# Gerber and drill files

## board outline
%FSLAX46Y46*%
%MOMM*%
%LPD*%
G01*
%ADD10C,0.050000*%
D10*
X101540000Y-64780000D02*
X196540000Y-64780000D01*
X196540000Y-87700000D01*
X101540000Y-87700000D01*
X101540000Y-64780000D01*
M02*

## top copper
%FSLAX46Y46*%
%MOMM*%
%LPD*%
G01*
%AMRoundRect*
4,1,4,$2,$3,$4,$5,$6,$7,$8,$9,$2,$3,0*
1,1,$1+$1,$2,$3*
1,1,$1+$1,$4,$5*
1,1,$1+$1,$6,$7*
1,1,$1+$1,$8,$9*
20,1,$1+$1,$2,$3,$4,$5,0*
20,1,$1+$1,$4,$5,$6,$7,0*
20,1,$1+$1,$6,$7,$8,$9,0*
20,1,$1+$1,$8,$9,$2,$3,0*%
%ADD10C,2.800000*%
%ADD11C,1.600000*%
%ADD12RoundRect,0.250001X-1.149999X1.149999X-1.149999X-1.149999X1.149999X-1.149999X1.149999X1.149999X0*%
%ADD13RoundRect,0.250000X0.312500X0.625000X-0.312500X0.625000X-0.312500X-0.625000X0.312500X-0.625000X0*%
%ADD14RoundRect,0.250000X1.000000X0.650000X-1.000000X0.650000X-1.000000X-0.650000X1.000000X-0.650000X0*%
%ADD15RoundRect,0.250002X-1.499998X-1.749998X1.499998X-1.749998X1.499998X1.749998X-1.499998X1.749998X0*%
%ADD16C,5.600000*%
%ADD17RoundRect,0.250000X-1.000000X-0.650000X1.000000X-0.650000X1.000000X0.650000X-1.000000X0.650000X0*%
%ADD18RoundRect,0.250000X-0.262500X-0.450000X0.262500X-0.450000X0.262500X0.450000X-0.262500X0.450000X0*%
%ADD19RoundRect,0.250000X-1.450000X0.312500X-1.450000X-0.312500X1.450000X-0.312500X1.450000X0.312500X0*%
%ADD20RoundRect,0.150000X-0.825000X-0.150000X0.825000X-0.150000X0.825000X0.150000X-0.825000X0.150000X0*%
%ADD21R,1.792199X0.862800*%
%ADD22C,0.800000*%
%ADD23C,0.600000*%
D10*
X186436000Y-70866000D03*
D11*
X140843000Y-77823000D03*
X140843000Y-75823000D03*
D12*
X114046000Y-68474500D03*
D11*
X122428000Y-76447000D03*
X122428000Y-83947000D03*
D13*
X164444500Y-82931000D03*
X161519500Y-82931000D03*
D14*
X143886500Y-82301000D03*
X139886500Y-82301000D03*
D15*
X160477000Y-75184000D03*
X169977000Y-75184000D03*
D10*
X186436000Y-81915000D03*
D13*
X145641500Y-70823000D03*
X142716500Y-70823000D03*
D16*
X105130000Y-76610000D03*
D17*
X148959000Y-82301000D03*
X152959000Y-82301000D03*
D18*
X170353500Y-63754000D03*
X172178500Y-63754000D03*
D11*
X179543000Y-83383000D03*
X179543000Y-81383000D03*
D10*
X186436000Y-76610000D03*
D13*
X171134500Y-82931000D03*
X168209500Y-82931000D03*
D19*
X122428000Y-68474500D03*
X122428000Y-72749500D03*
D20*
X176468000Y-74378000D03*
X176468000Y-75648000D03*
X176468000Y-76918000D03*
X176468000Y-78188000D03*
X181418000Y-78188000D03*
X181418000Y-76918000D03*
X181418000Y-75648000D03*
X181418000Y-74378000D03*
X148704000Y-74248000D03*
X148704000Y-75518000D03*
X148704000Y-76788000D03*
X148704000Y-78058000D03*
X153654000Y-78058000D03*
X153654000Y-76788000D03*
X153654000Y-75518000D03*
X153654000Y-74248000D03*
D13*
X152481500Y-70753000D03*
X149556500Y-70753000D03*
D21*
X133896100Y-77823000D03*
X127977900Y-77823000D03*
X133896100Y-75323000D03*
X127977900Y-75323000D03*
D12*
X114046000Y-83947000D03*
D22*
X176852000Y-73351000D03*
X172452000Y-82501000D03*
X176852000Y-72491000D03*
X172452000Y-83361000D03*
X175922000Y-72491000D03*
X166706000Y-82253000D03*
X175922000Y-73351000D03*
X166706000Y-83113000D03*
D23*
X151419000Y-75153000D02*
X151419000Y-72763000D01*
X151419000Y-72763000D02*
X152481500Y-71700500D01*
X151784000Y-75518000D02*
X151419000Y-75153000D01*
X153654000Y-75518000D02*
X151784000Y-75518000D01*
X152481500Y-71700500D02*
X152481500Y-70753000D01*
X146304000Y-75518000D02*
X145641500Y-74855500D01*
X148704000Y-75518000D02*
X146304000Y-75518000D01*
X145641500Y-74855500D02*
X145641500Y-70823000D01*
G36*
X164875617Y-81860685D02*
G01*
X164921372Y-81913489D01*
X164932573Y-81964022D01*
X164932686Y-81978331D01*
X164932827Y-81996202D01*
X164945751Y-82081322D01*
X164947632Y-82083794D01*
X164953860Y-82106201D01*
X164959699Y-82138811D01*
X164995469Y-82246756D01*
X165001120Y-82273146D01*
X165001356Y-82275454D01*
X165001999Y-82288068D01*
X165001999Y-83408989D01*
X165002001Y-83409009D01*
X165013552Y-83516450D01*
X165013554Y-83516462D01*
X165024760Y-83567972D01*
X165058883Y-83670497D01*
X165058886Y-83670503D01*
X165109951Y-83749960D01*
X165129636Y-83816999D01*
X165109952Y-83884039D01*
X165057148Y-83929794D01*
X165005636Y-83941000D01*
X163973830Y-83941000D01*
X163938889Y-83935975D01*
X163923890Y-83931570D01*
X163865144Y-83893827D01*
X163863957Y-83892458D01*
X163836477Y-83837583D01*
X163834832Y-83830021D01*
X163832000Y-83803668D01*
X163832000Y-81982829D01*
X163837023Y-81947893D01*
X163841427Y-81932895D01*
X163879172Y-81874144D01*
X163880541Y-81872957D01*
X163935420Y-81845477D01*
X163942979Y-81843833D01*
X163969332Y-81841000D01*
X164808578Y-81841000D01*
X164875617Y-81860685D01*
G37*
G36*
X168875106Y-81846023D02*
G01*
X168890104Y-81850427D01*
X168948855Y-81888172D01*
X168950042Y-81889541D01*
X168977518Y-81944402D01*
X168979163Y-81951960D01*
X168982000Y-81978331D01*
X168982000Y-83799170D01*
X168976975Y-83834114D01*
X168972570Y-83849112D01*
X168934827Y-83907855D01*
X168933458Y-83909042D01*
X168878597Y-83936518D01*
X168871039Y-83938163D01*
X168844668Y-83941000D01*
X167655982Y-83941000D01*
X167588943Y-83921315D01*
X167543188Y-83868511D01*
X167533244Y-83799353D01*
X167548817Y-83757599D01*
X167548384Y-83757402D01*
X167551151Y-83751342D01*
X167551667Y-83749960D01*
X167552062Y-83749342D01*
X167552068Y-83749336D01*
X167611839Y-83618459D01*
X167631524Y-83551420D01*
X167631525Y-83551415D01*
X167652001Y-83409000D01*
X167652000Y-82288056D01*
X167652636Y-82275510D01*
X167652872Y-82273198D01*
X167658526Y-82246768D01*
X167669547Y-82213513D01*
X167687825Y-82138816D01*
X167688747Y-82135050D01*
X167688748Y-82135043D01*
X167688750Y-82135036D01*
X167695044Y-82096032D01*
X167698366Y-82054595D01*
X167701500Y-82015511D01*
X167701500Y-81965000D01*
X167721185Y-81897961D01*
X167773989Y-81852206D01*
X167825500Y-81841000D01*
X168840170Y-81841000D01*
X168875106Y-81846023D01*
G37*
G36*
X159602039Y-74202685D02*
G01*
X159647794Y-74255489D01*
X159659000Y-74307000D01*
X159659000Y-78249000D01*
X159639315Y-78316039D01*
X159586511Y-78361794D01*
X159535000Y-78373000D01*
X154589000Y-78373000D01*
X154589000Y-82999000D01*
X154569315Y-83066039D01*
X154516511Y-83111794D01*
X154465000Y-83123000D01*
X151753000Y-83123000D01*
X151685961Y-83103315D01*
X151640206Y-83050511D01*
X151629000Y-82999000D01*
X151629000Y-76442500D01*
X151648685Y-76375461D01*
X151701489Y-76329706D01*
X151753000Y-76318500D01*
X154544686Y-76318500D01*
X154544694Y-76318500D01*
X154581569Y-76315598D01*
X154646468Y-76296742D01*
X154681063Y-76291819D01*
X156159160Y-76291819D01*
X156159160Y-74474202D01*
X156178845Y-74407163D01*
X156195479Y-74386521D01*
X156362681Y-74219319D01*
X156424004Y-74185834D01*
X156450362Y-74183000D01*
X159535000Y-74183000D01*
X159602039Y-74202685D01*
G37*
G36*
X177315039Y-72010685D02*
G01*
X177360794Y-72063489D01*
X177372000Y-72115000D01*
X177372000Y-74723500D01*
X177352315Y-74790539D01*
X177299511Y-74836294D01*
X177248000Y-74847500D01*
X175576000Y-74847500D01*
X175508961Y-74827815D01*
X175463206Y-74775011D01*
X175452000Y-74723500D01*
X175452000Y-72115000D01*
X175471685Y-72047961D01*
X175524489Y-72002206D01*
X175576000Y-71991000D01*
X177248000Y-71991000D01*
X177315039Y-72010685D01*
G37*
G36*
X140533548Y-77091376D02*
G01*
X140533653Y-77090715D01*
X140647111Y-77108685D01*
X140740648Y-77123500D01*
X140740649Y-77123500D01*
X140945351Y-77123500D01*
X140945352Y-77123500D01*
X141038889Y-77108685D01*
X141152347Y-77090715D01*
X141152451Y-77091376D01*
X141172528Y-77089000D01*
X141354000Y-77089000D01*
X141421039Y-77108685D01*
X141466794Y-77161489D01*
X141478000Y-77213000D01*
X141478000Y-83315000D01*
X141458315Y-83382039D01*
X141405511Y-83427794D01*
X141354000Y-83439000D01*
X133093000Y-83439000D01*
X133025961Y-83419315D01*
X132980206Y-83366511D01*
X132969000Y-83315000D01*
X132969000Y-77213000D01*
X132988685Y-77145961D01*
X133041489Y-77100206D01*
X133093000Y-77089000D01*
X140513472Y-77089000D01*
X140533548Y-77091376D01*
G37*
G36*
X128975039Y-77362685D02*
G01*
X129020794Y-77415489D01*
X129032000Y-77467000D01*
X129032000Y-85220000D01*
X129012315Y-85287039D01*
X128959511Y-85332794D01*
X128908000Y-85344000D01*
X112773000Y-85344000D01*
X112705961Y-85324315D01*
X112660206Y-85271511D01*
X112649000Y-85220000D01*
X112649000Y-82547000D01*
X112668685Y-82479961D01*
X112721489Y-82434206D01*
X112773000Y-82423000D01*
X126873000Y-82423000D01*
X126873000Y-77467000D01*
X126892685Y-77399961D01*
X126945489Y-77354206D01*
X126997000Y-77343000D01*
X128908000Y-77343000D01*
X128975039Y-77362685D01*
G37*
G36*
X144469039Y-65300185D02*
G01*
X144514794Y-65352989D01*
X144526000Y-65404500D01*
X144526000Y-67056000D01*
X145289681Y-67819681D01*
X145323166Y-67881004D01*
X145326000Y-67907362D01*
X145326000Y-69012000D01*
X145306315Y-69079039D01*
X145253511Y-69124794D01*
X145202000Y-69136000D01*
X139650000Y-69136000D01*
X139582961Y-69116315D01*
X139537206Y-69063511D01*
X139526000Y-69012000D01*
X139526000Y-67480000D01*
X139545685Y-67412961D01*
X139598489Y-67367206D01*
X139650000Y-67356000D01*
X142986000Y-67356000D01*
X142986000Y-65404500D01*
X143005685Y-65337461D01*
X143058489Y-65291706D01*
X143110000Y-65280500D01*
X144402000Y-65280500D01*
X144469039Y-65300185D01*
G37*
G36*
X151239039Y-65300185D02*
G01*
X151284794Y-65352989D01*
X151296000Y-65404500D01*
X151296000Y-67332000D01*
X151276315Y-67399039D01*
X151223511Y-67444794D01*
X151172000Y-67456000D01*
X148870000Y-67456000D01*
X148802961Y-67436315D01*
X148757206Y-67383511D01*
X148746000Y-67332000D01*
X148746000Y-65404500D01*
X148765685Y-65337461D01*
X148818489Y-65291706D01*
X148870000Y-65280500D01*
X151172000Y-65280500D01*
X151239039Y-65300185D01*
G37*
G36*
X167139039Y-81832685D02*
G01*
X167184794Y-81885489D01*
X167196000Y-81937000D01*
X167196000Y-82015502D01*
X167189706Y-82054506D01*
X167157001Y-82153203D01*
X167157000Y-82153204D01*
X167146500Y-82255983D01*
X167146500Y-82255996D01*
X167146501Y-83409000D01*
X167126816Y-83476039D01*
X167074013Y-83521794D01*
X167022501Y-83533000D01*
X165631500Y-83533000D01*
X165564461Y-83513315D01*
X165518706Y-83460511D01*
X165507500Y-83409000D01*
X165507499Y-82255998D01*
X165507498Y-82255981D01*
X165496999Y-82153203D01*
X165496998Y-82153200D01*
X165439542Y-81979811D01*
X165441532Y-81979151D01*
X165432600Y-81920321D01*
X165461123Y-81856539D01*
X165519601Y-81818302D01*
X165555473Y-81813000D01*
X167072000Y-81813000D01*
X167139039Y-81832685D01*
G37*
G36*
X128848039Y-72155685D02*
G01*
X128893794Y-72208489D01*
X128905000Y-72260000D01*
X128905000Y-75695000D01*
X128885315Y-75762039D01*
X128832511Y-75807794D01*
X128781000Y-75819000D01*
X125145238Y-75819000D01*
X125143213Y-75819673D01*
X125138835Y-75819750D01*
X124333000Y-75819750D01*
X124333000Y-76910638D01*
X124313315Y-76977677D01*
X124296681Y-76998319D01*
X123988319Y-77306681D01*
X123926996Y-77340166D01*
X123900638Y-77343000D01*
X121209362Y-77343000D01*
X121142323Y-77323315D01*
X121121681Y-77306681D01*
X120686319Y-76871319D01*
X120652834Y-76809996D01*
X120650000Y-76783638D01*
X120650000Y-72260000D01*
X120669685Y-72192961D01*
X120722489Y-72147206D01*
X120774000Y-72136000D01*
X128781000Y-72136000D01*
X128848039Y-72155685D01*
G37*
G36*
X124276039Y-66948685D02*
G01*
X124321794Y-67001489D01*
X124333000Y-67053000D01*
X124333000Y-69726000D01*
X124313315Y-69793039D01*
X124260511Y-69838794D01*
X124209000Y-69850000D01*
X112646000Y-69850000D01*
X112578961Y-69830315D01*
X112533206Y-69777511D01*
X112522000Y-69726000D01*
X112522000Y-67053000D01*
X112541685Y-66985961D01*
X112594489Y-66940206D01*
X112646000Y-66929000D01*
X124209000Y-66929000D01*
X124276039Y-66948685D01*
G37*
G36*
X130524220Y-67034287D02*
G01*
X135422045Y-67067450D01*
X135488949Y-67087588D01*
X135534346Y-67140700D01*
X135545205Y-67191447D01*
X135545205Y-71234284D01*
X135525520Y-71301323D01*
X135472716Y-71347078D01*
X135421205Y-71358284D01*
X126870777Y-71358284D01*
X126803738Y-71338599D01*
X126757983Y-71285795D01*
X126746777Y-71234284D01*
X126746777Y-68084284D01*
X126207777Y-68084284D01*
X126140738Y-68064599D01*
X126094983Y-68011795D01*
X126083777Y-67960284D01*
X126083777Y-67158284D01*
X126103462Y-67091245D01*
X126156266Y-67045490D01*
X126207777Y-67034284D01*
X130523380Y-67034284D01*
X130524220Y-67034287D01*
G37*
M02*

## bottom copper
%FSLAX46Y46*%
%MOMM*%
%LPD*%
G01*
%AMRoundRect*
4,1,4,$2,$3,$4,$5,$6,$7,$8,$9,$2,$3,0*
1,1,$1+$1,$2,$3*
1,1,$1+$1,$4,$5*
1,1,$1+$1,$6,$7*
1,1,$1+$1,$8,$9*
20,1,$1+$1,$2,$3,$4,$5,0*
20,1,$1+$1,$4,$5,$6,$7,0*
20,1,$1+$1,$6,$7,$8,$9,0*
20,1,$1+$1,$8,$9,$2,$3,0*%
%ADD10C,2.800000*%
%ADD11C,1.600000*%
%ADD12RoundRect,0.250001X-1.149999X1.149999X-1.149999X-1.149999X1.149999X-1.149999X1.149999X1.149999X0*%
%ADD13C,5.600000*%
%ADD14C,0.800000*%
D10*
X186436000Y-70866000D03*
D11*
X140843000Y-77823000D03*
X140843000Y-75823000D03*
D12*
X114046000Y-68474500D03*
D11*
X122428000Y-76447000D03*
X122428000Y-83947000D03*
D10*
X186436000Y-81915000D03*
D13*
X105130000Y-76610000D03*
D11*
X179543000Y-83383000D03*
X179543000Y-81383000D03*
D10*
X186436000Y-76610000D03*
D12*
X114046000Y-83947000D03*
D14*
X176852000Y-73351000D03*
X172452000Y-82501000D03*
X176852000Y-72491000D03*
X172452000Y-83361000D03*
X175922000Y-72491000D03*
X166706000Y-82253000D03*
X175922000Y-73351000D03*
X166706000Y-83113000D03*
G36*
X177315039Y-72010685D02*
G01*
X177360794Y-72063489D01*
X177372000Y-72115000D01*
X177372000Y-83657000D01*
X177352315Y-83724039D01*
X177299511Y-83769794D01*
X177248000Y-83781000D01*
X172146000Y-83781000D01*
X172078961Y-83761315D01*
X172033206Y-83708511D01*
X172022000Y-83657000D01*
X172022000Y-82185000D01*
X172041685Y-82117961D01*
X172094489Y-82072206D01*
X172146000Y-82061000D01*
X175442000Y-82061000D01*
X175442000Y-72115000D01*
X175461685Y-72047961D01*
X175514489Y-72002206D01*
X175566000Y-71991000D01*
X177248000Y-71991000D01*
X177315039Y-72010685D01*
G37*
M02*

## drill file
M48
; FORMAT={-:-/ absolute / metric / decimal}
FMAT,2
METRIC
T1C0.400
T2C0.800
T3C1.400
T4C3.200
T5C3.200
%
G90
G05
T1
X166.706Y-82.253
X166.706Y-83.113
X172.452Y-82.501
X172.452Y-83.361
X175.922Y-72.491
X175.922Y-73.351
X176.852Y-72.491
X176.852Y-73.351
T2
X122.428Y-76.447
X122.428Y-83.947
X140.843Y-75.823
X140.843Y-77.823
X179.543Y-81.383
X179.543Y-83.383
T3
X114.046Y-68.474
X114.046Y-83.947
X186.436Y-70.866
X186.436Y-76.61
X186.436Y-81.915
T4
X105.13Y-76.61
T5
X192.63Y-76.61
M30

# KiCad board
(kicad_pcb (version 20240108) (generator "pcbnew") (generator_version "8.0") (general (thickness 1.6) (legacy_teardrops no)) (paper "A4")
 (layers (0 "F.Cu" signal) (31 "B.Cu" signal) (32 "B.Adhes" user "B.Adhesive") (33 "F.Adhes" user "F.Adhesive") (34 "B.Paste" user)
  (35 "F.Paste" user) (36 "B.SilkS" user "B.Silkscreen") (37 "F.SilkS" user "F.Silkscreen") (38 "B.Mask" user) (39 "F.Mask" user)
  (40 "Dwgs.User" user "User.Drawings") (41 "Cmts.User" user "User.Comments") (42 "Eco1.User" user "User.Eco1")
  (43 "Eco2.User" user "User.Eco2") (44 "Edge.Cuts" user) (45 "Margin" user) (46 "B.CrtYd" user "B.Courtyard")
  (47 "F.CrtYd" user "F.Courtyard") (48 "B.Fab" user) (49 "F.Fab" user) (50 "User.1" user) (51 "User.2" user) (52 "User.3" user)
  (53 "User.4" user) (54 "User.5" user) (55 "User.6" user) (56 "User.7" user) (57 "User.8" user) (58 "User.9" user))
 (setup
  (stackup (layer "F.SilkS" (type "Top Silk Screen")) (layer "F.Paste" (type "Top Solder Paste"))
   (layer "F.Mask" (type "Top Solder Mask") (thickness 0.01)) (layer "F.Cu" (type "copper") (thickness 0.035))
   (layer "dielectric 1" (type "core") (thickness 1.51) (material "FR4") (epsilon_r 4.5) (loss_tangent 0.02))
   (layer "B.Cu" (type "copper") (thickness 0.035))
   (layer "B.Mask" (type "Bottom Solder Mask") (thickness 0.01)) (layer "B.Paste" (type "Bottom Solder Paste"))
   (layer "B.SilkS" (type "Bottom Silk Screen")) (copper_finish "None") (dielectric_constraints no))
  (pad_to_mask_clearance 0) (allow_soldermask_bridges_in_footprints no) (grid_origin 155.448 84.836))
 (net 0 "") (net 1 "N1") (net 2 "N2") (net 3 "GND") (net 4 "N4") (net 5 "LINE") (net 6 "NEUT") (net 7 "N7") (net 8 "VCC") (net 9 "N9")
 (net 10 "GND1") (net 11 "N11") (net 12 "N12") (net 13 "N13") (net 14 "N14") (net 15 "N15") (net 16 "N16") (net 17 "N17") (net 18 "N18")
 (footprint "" (layer "F.Cu") (at 186.436 70.866)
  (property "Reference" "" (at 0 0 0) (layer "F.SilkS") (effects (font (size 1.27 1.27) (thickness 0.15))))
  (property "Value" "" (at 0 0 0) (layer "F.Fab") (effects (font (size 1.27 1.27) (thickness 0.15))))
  (pad "2" thru_hole circle (at 0 0 270) (size 2.8 2.8) (drill 1.4) (layers "*.Cu" "*.Mask") (remove_unused_layers no) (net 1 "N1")))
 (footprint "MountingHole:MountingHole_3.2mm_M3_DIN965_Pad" (layer "F.Cu") (at 192.63 76.61 90)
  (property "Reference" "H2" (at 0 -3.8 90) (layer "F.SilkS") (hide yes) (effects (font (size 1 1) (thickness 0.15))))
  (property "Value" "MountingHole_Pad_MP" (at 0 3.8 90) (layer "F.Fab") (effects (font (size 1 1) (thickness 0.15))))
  (pad "" np_thru_hole circle (at 0 0 90) (size 3.2 3.2) (drill 3.2) (layers "F&B.Cu" "*.Mask")))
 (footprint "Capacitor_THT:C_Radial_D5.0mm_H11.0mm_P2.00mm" (layer "F.Cu") (at 140.843 77.823 90)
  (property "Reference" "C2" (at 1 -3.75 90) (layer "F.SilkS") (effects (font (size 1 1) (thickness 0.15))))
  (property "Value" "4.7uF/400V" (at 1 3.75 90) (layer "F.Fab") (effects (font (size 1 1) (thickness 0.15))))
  (pad "1" thru_hole circle (at 0 0 90) (size 1.6 1.6) (drill 0.8) (layers "*.Cu" "*.Mask") (remove_unused_layers no) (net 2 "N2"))
  (pad "2" thru_hole circle (at 2 0 90) (size 1.6 1.6) (drill 0.8) (layers "*.Cu" "*.Mask") (remove_unused_layers no) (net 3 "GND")))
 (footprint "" (layer "F.Cu") (at 114.046 68.4745)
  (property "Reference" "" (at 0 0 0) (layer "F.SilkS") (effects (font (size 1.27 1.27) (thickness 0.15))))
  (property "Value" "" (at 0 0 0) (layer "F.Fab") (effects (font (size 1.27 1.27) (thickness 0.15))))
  (pad "1" thru_hole roundrect (at 0 0 270) (size 2.8 2.8) (drill 1.4) (layers "*.Cu" "*.Mask") (remove_unused_layers no)
   (roundrect_rratio 0.089286) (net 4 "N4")))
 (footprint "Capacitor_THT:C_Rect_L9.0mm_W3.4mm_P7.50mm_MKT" (layer "F.Cu") (at 122.428 76.447 -90)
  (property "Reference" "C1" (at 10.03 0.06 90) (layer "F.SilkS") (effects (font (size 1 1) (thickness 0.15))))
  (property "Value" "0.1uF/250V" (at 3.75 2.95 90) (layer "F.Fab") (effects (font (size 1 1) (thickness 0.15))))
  (pad "1" thru_hole circle (at 0 0 270) (size 1.6 1.6) (drill 0.8) (layers "*.Cu" "*.Mask") (remove_unused_layers no) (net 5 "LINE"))
  (pad "2" thru_hole circle (at 7.5 0 270) (size 1.6 1.6) (drill 0.8) (layers "*.Cu" "*.Mask") (remove_unused_layers no) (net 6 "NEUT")))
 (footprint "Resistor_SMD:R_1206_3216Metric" (layer "F.Cu") (at 162.982 82.931 180)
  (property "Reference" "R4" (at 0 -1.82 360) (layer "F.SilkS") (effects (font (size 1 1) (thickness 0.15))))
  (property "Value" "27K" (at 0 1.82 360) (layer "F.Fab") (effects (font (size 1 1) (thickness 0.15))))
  (pad "1" smd roundrect (at -1.4625 0 180) (size 1.125 1.75) (layers "F.Cu" "F.Paste" "F.Mask") (roundrect_rratio 0.222222) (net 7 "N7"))
  (pad "2" smd roundrect (at 1.4625 0 180) (size 1.125 1.75) (layers "F.Cu" "F.Paste" "F.Mask") (roundrect_rratio 0.222222) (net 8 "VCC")))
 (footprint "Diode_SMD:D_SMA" (layer "F.Cu") (at 141.8865 82.301 180)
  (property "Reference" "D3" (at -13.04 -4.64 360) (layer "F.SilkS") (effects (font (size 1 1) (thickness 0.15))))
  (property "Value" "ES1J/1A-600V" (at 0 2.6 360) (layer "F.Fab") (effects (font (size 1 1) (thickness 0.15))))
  (pad "1" smd roundrect (at -2 0 180) (size 2.5 1.8) (layers "F.Cu" "F.Paste" "F.Mask") (roundrect_rratio 0.1388888889) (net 8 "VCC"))
  (pad "2" smd roundrect (at 2 0 180) (size 2.5 1.8) (layers "F.Cu" "F.Paste" "F.Mask") (roundrect_rratio 0.1388888889) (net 2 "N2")))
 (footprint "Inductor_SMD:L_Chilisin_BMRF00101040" (layer "F.Cu") (at 165.227 75.184)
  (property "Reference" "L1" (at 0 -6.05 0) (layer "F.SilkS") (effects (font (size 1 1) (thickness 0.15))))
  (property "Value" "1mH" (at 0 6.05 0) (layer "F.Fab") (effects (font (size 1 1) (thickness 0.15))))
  (pad "1" smd roundrect (at -4.75 0) (size 3.5 4) (layers "F.Cu" "F.Paste" "F.Mask") (roundrect_rratio 0.071429) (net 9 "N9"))
  (pad "2" smd roundrect (at 4.75 0) (size 3.5 4) (layers "F.Cu" "F.Paste" "F.Mask") (roundrect_rratio 0.071429) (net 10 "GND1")))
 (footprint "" (layer "F.Cu") (at 186.436 81.915)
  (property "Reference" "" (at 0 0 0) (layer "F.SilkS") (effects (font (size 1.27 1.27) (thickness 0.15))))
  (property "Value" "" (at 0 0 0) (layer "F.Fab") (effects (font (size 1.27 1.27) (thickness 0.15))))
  (pad "2" thru_hole circle (at 0 0 270) (size 2.8 2.8) (drill 1.4) (layers "*.Cu" "*.Mask") (remove_unused_layers no)))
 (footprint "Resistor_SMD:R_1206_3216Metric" (layer "F.Cu") (at 144.179 70.823 180)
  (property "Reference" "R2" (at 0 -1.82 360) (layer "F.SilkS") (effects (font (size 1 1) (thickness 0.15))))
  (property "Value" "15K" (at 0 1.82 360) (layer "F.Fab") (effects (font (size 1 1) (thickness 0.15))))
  (pad "1" smd roundrect (at -1.4625 0 180) (size 1.125 1.75) (layers "F.Cu" "F.Paste" "F.Mask") (roundrect_rratio 0.222222) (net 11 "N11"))
  (pad "2" smd roundrect (at 1.4625 0 180) (size 1.125 1.75) (layers "F.Cu" "F.Paste" "F.Mask") (roundrect_rratio 0.222222) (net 3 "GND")))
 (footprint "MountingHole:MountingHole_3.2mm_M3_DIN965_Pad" (layer "F.Cu") (at 105.13 76.61)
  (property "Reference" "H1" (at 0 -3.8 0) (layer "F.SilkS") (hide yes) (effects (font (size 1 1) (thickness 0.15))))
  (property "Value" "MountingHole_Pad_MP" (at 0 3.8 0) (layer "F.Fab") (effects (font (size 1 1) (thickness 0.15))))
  (pad "1" thru_hole circle (at 0 0) (size 5.6 5.6) (drill 3.2) (layers "*.Cu" "*.Mask") (remove_unused_layers no)))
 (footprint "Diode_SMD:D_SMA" (layer "F.Cu") (at 150.959 82.301)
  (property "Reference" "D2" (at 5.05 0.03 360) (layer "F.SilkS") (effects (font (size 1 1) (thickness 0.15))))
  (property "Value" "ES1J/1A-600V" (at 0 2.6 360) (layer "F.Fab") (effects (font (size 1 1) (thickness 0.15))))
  (pad "1" smd roundrect (at -2 0) (size 2.5 1.8) (layers "F.Cu" "F.Paste" "F.Mask") (roundrect_rratio 0.1388888889) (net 8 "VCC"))
  (pad "2" smd roundrect (at 2 0) (size 2.5 1.8) (layers "F.Cu" "F.Paste" "F.Mask") (roundrect_rratio 0.1388888889) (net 9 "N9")))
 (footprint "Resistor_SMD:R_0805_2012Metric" (layer "F.Cu") (at 171.266 63.754)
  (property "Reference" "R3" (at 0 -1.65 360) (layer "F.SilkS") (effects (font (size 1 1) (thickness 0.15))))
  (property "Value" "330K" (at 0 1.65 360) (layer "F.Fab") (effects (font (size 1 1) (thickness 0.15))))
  (pad "1" smd roundrect (at -0.9125 0) (size 1.025 1.4) (layers "F.Cu" "F.Paste" "F.Mask") (roundrect_rratio 0.243902) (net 9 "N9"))
  (pad "2" smd roundrect (at 0.9125 0) (size 1.025 1.4) (layers "F.Cu" "F.Paste" "F.Mask") (roundrect_rratio 0.243902) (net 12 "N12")))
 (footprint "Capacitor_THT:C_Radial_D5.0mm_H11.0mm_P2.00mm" (layer "F.Cu") (at 179.543 83.383 90)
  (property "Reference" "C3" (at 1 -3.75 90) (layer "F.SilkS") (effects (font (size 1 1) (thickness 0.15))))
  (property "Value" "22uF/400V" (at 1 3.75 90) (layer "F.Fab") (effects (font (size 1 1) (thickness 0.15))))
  (pad "1" thru_hole circle (at 0 0 90) (size 1.6 1.6) (drill 0.8) (layers "*.Cu" "*.Mask") (remove_unused_layers no) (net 8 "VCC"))
  (pad "2" thru_hole circle (at 2 0 90) (size 1.6 1.6) (drill 0.8) (layers "*.Cu" "*.Mask") (remove_unused_layers no) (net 10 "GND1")))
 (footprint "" (layer "F.Cu") (at 186.436 76.61)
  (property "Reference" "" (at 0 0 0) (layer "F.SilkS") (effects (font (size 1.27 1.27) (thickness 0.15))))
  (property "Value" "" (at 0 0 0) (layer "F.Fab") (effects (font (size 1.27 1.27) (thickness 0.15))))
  (pad "2" thru_hole circle (at 0 0 270) (size 2.8 2.8) (drill 1.4) (layers "*.Cu" "*.Mask") (remove_unused_layers no)))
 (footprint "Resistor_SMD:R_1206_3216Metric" (layer "F.Cu") (at 169.672 82.931 180)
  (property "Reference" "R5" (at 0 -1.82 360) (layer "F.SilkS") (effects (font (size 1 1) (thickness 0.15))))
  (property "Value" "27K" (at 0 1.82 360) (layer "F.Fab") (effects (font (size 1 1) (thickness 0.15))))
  (pad "1" smd roundrect (at -1.4625 0 180) (size 1.125 1.75) (layers "F.Cu" "F.Paste" "F.Mask") (roundrect_rratio 0.222222) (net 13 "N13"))
  (pad "2" smd roundrect (at 1.4625 0 180) (size 1.125 1.75) (layers "F.Cu" "F.Paste" "F.Mask") (roundrect_rratio 0.222222) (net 7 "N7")))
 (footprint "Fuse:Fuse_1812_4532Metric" (layer "F.Cu") (at 122.428 70.612 -90)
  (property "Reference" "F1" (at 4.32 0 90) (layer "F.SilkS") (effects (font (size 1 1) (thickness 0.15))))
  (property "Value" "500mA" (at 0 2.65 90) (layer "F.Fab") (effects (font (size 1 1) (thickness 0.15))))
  (pad "1" smd roundrect (at -2.1375 0 270) (size 1.125 3.4) (layers "F.Cu" "F.Paste" "F.Mask") (roundrect_rratio 0.222222) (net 4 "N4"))
  (pad "2" smd roundrect (at 2.1375 0 270) (size 1.125 3.4) (layers "F.Cu" "F.Paste" "F.Mask") (roundrect_rratio 0.222222) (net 5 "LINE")))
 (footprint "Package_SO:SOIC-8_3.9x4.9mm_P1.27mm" (layer "F.Cu") (at 178.943 76.283)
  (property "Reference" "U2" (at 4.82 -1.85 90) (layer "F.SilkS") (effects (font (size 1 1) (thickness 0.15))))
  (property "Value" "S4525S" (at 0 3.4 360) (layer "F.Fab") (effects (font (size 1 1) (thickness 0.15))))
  (pad "1" smd roundrect (at -2.475 -1.905) (size 1.95 0.6) (layers "F.Cu" "F.Paste" "F.Mask") (roundrect_rratio 0.25) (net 13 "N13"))
  (pad "2" smd roundrect (at -2.475 -0.635) (size 1.95 0.6) (layers "F.Cu" "F.Paste" "F.Mask") (roundrect_rratio 0.25) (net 12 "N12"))
  (pad "3" smd roundrect (at -2.475 0.635) (size 1.95 0.6) (layers "F.Cu" "F.Paste" "F.Mask") (roundrect_rratio 0.25) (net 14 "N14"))
  (pad "4" smd roundrect (at -2.475 1.905) (size 1.95 0.6) (layers "F.Cu" "F.Paste" "F.Mask") (roundrect_rratio 0.25) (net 10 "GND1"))
  (pad "5" smd roundrect (at 2.475 1.905) (size 1.95 0.6) (layers "F.Cu" "F.Paste" "F.Mask") (roundrect_rratio 0.25) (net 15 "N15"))
  (pad "6" smd roundrect (at 2.475 0.635) (size 1.95 0.6) (layers "F.Cu" "F.Paste" "F.Mask") (roundrect_rratio 0.25) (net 15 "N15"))
  (pad "7" smd roundrect (at 2.475 -0.635) (size 1.95 0.6) (layers "F.Cu" "F.Paste" "F.Mask") (roundrect_rratio 0.25) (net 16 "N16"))
  (pad "8" smd roundrect (at 2.475 -1.905) (size 1.95 0.6) (layers "F.Cu" "F.Paste" "F.Mask") (roundrect_rratio 0.25) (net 16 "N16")))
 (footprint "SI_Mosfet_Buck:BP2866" (layer "F.Cu") (at 151.179 76.153)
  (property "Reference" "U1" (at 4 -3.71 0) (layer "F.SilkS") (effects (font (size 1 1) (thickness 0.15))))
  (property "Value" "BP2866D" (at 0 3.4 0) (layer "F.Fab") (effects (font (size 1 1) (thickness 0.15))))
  (pad "1" smd roundrect (at -2.475 -1.905) (size 1.95 0.6) (layers "F.Cu" "F.Paste" "F.Mask") (roundrect_rratio 0.25) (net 3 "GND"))
  (pad "2" smd roundrect (at -2.475 -0.635) (size 1.95 0.6) (layers "F.Cu" "F.Paste" "F.Mask") (roundrect_rratio 0.25) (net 11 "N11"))
  (pad "3" smd roundrect (at -2.475 0.635) (size 1.95 0.6) (layers "F.Cu" "F.Paste" "F.Mask") (roundrect_rratio 0.25) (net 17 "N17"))
  (pad "4" smd roundrect (at -2.475 1.905) (size 1.95 0.6) (layers "F.Cu" "F.Paste" "F.Mask") (roundrect_rratio 0.25) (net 8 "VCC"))
  (pad "5" smd roundrect (at 2.475 1.905) (size 1.95 0.6) (layers "F.Cu" "F.Paste" "F.Mask") (roundrect_rratio 0.25) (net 9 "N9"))
  (pad "6" smd roundrect (at 2.475 0.635) (size 1.95 0.6) (layers "F.Cu" "F.Paste" "F.Mask") (roundrect_rratio 0.25) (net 9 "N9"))
  (pad "7" smd roundrect (at 2.475 -0.635) (size 1.95 0.6) (layers "F.Cu" "F.Paste" "F.Mask") (roundrect_rratio 0.25) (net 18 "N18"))
  (pad "8" smd roundrect (at 2.475 -1.905) (size 1.95 0.6) (layers "F.Cu" "F.Paste" "F.Mask") (roundrect_rratio 0.25)))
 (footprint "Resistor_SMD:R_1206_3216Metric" (layer "F.Cu") (at 151.019 70.753 180)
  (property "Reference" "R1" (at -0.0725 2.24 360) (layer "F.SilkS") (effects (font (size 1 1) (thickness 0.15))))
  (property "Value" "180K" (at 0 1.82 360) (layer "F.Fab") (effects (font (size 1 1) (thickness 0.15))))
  (pad "1" smd roundrect (at -1.4625 0 180) (size 1.125 1.75) (layers "F.Cu" "F.Paste" "F.Mask") (roundrect_rratio 0.222222) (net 18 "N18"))
  (pad "2" smd roundrect (at 1.4625 0 180) (size 1.125 1.75) (layers "F.Cu" "F.Paste" "F.Mask") (roundrect_rratio 0.222222) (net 3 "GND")))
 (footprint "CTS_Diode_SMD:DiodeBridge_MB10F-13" (layer "F.Cu") (at 130.937 76.573 180)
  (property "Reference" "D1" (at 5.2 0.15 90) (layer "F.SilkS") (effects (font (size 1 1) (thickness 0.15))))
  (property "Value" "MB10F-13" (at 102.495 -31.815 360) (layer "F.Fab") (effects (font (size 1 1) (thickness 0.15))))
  (pad "1" smd rect (at -2.9591 -1.25 180) (size 1.792199 0.8628) (layers "F.Cu" "F.Paste" "F.Mask") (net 2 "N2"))
  (pad "2" smd rect (at 2.9591 -1.25 180) (size 1.792199 0.8628) (layers "F.Cu" "F.Paste" "F.Mask") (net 6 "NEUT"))
  (pad "3" smd rect (at -2.9591 1.25 180) (size 1.792199 0.8628) (layers "F.Cu" "F.Paste" "F.Mask") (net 3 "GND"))
  (pad "4" smd rect (at 2.9591 1.25 180) (size 1.792199 0.8628) (layers "F.Cu" "F.Paste" "F.Mask") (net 5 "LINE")))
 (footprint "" (layer "F.Cu") (at 114.046 83.947)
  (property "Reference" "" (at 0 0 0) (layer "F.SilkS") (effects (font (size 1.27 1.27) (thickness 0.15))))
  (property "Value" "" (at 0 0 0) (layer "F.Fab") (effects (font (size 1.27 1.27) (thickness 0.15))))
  (pad "1" thru_hole roundrect (at 0 0 270) (size 2.8 2.8) (drill 1.4) (layers "*.Cu" "*.Mask") (remove_unused_layers no)
   (roundrect_rratio 0.089286) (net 6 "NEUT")))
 (gr_rect (start 101.54 64.78) (end 196.54 87.7) (stroke (width 0.05) (type default)) (fill none) (layer "Edge.Cuts"))
 (segment (start 151.419 75.153) (end 151.419 72.763) (width 0.6) (layer "F.Cu") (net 18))
 (segment (start 151.419 72.763) (end 152.4815 71.7005) (width 0.6) (layer "F.Cu") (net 18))
 (segment (start 151.784 75.518) (end 151.419 75.153) (width 0.6) (layer "F.Cu") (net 18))
 (segment (start 153.654 75.518) (end 151.784 75.518) (width 0.6) (layer "F.Cu") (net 18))
 (segment (start 152.4815 71.7005) (end 152.4815 70.753) (width 0.6) (layer "F.Cu") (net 18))
 (segment (start 146.304 75.518) (end 145.6415 74.8555) (width 0.6) (layer "F.Cu") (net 11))
 (segment (start 148.704 75.518) (end 146.304 75.518) (width 0.6) (layer "F.Cu") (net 11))
 (segment (start 145.6415 74.8555) (end 145.6415 70.823) (width 0.6) (layer "F.Cu") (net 11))
 (via (at 176.852 73.351) (size 0.8) (drill 0.4) (layers "F.Cu" "B.Cu") (free yes) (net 13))
 (via (at 172.452 82.501) (size 0.8) (drill 0.4) (layers "F.Cu" "B.Cu") (free yes) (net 13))
 (via (at 176.852 72.491) (size 0.8) (drill 0.4) (layers "F.Cu" "B.Cu") (free yes)
  (teardrops (best_length_ratio 0.5) (max_length 1) (best_width_ratio 1) (max_width 2) (curve_points 5) (filter_ratio 0.9) (enabled no)
   (allow_two_segments yes) (prefer_zone_connections yes))
  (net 13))
 (via (at 172.452 83.361) (size 0.8) (drill 0.4) (layers "F.Cu" "B.Cu") (free yes) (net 13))
 (via (at 175.922 72.491) (size 0.8) (drill 0.4) (layers "F.Cu" "B.Cu") (free yes) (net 13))
 (via (at 166.706 82.253) (size 0.8) (drill 0.4) (layers "F.Cu" "B.Cu") (free yes) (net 13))
 (via (at 175.922 73.351) (size 0.8) (drill 0.4) (layers "F.Cu" "B.Cu") (free yes) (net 13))
 (via (at 166.706 83.113) (size 0.8) (drill 0.4) (layers "F.Cu" "B.Cu") (free yes) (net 13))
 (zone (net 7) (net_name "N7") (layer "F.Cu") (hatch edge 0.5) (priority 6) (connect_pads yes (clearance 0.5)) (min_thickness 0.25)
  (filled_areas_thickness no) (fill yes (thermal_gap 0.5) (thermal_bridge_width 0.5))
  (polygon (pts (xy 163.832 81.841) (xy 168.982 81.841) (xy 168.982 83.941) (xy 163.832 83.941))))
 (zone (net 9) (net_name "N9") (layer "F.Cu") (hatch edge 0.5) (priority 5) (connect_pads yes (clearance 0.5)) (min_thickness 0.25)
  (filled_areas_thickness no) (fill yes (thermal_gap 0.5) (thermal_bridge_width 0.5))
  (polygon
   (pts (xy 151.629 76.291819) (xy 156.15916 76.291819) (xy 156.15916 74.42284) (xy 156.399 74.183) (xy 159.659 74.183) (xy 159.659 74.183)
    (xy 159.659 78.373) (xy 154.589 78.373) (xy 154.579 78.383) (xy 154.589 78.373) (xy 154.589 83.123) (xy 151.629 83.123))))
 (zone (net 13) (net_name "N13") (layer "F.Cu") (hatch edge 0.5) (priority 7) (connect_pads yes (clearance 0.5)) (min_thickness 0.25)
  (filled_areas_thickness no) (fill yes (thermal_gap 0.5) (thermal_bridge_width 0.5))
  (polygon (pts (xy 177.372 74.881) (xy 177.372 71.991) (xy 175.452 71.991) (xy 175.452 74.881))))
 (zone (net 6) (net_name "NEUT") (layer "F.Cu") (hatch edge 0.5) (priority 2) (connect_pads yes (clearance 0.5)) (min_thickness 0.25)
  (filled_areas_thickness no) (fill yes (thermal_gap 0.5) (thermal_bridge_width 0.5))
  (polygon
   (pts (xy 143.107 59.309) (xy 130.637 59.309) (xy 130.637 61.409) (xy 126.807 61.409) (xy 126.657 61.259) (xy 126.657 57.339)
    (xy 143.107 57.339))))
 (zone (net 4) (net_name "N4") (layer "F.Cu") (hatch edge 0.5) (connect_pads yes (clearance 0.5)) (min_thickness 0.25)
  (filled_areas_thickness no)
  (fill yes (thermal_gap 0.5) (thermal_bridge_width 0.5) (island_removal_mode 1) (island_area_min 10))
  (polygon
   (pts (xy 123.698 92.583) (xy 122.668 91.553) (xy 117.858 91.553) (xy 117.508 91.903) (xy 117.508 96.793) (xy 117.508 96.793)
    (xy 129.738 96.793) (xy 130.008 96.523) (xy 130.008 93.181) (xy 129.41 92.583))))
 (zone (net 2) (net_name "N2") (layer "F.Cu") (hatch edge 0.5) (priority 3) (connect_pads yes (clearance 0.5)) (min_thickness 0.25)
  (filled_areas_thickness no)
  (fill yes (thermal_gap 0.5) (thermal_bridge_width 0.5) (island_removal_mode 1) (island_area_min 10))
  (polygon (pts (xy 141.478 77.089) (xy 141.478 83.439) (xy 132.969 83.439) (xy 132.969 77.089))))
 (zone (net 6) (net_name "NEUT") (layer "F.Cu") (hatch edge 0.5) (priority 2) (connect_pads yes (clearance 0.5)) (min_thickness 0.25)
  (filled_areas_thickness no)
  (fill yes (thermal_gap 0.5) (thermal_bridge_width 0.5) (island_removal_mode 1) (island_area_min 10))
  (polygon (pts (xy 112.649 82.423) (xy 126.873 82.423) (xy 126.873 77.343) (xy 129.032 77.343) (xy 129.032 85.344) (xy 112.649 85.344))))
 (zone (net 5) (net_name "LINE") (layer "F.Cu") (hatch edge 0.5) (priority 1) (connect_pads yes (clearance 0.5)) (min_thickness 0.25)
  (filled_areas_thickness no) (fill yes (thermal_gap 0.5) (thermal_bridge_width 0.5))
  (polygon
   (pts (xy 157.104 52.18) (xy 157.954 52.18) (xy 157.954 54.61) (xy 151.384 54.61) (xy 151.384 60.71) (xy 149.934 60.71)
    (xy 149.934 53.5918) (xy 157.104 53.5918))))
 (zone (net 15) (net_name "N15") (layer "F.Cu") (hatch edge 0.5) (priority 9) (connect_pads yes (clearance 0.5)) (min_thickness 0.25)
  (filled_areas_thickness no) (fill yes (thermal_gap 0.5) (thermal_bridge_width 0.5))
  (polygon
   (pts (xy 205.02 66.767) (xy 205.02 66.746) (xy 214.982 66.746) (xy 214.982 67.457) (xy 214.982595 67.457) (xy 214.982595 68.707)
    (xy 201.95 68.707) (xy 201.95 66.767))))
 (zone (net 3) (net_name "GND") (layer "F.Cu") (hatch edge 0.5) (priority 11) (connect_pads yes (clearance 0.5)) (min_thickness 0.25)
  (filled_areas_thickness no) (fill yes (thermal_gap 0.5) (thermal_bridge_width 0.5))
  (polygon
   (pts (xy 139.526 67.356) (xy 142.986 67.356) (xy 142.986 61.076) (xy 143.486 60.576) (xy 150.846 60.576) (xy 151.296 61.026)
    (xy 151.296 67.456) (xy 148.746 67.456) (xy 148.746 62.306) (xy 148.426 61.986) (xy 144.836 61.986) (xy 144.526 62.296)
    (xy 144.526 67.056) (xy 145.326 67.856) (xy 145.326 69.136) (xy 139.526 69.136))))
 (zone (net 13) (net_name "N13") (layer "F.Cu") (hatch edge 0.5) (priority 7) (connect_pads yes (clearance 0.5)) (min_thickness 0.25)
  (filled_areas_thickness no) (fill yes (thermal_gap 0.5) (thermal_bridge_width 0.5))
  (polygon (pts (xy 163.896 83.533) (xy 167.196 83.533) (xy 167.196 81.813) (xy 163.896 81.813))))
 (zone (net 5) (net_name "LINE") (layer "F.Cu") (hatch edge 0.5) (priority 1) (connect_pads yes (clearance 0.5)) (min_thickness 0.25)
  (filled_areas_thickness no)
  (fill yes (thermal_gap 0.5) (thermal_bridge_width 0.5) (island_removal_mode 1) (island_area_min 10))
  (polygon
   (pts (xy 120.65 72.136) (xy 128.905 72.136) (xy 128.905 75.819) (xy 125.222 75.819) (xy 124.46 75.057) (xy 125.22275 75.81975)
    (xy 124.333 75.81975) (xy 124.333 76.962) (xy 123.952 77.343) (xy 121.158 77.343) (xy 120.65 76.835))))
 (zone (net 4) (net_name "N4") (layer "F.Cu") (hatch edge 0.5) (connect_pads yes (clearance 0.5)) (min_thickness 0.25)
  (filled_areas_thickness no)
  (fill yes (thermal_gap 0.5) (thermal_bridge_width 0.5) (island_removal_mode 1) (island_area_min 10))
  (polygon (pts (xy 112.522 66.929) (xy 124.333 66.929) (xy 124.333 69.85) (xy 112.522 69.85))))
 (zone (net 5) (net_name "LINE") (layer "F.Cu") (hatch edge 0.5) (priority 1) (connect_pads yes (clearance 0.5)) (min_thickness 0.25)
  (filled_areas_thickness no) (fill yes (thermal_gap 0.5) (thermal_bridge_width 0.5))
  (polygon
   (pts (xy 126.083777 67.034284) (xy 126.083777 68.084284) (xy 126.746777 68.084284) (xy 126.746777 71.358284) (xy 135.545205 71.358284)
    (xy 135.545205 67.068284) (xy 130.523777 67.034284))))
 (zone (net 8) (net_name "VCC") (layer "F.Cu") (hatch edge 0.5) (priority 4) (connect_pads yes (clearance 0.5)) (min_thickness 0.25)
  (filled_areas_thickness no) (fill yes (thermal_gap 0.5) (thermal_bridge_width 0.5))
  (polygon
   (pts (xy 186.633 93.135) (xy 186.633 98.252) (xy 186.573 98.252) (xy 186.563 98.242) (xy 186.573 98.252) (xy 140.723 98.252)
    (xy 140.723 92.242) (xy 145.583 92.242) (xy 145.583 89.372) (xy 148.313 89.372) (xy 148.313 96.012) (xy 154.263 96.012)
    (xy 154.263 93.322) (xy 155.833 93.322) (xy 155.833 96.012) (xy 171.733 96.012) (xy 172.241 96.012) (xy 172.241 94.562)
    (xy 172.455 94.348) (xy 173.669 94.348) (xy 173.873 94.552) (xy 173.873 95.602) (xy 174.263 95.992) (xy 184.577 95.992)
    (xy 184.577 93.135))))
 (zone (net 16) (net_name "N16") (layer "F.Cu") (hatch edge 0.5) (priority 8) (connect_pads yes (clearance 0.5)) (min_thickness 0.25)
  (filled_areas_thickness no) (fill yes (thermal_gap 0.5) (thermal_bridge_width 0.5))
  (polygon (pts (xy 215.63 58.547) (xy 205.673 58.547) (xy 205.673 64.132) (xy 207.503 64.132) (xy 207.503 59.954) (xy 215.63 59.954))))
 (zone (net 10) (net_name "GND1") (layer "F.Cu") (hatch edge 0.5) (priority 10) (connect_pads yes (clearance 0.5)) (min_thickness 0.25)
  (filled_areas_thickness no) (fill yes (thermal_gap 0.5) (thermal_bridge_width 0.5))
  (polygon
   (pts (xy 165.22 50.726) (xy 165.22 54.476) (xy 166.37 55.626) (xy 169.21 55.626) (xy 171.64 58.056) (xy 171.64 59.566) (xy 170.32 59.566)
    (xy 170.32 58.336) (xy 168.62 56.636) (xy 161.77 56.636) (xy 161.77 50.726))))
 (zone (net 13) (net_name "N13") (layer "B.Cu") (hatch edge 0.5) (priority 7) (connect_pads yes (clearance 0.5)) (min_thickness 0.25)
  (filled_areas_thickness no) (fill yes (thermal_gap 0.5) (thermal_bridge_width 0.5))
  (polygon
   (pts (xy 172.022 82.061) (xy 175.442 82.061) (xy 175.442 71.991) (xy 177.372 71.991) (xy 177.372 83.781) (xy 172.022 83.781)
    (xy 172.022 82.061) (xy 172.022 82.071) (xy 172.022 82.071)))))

